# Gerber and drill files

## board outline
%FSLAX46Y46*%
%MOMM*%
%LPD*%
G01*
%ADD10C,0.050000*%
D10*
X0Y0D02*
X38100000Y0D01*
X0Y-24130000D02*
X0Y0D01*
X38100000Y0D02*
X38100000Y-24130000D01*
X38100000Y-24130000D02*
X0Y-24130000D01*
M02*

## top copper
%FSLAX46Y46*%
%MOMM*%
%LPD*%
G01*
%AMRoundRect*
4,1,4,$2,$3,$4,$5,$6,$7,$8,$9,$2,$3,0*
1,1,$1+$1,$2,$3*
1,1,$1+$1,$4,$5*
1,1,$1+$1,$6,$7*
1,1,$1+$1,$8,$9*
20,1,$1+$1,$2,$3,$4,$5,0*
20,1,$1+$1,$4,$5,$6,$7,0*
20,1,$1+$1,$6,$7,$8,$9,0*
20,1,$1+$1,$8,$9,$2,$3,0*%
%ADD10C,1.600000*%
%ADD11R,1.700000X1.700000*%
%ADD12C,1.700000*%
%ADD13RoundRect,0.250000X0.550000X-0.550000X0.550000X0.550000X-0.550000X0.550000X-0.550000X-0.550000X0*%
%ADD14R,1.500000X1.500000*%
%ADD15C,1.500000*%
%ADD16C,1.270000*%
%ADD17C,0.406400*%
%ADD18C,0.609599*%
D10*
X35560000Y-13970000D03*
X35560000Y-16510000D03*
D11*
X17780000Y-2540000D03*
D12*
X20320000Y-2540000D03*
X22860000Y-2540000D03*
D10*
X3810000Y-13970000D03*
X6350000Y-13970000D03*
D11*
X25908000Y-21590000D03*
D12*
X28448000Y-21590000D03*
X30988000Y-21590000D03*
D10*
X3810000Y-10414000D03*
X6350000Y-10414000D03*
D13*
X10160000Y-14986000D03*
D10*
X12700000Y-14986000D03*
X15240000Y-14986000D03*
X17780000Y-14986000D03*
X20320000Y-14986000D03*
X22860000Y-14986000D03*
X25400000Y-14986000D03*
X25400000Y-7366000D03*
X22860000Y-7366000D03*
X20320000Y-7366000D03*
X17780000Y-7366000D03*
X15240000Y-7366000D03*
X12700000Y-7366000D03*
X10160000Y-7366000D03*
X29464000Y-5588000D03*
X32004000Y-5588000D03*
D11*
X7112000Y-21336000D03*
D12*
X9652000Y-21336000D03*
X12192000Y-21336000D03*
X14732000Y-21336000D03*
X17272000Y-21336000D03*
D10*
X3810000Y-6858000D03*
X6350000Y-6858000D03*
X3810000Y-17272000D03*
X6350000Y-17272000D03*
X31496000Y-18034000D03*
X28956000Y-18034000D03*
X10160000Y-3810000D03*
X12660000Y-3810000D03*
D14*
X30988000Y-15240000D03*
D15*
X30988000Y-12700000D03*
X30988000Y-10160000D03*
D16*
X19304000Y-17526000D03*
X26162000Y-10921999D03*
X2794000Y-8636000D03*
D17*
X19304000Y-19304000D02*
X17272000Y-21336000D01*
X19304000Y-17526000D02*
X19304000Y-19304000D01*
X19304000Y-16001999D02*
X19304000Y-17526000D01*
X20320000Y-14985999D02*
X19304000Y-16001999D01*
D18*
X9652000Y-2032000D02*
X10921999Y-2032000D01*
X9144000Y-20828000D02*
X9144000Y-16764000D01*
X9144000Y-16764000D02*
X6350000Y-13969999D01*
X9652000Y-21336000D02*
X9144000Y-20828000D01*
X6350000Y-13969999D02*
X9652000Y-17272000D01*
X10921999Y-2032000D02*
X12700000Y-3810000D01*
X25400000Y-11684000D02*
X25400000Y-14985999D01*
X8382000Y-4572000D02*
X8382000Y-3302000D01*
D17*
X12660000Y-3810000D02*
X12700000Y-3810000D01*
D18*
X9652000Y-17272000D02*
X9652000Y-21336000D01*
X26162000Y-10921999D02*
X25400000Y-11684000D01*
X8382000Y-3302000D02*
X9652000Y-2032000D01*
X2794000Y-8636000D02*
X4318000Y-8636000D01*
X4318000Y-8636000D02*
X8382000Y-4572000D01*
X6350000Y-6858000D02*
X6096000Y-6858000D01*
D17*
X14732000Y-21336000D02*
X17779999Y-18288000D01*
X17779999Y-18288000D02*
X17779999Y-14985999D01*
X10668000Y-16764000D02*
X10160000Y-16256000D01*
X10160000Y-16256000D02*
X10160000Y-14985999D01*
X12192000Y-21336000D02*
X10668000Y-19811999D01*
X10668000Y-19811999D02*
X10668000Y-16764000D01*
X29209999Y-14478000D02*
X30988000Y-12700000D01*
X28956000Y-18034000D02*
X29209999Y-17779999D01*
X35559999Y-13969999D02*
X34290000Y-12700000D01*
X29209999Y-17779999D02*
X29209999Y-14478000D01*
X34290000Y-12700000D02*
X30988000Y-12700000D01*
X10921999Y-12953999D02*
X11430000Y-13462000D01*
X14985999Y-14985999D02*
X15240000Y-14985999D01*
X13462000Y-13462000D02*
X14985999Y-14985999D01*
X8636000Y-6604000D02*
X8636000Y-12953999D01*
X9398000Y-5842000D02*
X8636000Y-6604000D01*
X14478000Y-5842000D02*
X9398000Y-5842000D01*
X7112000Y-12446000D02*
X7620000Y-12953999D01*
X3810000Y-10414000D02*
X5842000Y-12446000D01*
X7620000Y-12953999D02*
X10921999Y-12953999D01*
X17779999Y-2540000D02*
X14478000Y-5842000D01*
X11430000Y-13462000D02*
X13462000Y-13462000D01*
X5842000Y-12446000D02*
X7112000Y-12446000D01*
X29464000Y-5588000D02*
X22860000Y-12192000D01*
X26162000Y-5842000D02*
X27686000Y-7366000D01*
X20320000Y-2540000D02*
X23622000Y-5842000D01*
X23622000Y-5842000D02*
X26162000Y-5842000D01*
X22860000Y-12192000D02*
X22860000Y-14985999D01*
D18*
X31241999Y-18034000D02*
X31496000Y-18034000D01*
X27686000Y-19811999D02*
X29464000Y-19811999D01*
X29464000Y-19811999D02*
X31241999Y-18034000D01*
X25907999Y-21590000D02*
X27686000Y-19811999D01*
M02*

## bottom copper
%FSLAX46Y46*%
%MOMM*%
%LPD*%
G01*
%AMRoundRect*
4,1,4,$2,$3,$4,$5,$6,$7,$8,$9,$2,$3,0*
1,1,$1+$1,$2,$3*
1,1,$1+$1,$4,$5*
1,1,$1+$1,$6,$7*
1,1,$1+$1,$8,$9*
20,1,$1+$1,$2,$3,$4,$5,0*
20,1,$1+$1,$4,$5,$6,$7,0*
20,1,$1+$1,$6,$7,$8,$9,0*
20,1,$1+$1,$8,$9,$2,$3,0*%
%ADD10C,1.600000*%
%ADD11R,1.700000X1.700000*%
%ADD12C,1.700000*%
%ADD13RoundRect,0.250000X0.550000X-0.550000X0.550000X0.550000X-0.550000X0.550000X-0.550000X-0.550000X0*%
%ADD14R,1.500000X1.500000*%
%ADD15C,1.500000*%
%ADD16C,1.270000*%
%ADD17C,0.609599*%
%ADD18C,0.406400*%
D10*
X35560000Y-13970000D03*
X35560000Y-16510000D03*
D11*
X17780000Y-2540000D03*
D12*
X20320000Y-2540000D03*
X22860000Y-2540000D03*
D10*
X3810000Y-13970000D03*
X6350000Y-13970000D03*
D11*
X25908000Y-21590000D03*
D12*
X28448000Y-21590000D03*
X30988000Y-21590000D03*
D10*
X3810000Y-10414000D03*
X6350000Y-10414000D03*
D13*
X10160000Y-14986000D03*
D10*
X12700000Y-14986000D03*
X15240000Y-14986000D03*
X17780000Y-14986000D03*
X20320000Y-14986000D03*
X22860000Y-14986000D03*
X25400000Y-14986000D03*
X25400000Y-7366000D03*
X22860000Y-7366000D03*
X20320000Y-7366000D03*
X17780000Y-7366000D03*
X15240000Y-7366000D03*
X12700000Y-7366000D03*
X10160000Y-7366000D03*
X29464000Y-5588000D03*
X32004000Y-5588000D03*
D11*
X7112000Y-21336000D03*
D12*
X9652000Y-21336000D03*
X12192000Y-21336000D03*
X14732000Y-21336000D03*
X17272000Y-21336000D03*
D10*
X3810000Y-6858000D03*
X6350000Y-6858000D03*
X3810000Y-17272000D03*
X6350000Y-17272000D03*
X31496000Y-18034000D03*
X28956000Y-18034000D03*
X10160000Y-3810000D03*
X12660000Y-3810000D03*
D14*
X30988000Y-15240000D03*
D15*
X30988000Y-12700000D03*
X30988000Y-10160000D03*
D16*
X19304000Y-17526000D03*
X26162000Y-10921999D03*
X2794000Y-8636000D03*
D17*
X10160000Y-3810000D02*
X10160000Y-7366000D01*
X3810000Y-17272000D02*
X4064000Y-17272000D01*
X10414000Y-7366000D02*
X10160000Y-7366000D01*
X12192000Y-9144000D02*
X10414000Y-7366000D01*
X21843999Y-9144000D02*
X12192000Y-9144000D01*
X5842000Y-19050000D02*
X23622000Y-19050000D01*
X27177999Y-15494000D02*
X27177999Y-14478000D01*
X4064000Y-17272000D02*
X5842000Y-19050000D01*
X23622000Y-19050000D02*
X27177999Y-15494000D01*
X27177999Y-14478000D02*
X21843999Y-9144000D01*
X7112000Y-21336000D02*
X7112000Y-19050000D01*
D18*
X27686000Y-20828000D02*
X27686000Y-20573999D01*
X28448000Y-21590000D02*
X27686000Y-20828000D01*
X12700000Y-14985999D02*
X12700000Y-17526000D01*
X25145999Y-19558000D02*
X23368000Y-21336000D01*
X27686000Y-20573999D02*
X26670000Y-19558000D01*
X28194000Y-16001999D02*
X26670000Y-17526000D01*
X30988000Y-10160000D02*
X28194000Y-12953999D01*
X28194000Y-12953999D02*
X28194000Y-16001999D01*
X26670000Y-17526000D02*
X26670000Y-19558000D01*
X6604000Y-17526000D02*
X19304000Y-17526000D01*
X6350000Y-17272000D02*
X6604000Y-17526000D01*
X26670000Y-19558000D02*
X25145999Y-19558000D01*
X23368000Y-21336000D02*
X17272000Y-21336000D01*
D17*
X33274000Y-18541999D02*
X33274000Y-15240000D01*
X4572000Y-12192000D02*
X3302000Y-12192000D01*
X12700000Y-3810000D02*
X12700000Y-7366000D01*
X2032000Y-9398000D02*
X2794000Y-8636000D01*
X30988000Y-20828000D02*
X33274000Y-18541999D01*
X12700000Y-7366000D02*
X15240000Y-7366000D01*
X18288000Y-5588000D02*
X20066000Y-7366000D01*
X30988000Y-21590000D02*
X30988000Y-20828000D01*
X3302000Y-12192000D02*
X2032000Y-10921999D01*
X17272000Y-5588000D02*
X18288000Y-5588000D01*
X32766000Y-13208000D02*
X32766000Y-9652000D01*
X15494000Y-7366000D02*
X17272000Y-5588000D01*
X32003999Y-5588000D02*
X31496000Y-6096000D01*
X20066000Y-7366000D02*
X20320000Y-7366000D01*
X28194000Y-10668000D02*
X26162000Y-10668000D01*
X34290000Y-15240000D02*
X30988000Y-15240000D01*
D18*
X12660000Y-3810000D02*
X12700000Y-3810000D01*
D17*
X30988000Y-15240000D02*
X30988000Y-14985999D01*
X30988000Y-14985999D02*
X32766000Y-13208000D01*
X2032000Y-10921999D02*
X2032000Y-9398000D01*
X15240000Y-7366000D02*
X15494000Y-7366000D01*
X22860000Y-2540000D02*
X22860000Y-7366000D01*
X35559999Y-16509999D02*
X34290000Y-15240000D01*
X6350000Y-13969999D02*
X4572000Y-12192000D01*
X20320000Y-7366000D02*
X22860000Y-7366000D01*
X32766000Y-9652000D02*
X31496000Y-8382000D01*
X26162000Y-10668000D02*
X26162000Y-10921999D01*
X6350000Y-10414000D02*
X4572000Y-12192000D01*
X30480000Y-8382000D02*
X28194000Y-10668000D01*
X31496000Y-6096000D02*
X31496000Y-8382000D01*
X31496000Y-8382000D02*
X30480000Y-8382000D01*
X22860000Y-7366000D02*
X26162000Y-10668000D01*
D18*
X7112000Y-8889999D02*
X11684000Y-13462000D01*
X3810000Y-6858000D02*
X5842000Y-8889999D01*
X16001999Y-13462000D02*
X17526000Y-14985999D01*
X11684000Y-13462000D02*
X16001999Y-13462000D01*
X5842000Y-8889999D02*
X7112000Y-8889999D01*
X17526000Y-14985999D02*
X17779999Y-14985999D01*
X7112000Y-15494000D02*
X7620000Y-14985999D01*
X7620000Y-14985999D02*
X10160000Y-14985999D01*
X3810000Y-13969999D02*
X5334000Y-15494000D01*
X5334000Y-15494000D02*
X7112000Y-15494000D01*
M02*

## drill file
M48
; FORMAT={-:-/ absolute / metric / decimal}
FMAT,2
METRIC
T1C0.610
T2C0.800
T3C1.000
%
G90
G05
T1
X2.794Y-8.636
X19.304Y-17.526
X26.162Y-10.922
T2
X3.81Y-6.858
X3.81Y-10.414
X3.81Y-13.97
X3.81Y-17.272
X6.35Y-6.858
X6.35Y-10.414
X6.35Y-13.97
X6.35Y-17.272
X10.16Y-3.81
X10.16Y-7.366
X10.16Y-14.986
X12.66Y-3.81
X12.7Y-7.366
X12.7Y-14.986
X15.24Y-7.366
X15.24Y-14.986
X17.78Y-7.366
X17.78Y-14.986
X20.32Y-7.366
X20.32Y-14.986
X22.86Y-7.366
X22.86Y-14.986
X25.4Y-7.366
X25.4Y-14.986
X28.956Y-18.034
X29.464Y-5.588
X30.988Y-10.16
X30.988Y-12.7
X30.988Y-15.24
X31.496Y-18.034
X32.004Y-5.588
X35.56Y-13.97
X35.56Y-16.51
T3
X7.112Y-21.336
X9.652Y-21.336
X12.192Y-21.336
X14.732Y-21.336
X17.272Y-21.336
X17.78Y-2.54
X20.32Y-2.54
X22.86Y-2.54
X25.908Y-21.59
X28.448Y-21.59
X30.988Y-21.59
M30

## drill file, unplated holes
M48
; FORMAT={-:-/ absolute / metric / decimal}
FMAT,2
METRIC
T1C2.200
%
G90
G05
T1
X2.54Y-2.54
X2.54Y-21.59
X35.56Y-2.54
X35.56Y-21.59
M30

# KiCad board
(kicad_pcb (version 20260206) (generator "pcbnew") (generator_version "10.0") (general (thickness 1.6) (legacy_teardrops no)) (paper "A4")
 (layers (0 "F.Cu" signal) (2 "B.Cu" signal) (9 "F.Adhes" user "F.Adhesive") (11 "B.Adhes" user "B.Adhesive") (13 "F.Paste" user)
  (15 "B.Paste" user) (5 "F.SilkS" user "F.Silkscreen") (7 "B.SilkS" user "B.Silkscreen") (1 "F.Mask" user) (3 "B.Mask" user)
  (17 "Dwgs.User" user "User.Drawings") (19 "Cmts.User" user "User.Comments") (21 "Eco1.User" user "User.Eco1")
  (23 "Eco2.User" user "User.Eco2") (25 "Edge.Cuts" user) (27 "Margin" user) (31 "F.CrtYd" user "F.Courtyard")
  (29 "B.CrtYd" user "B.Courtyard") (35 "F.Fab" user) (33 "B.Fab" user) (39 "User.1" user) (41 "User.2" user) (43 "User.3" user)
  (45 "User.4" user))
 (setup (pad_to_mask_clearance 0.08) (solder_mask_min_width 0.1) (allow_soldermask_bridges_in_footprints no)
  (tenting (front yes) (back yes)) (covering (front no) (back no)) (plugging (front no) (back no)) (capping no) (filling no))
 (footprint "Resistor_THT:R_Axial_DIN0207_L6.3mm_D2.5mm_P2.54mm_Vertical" (layer "F.Cu") (at 35.56 13.97 -90)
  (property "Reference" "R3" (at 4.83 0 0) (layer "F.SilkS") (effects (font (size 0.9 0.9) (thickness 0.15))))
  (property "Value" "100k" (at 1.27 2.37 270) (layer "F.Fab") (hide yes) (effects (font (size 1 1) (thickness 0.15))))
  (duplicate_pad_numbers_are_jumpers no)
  (pad "1" thru_hole circle (at 0 0 270) (size 1.6 1.6) (drill 0.8) (layers "*.Cu" "*.Mask") (remove_unused_layers no) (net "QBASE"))
  (pad "2" thru_hole circle (at 2.54 0 270) (size 1.6 1.6) (drill 0.8) (layers "*.Cu" "*.Mask") (remove_unused_layers no) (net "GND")))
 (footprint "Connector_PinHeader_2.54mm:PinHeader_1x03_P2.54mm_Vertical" (layer "F.Cu") (at 17.78 2.54 90)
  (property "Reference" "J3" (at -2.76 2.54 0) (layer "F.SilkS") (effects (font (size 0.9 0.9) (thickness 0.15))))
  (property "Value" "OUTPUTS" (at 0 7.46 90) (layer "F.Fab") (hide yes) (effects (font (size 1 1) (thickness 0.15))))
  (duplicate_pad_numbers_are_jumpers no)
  (pad "1" thru_hole rect (at 0 0 90) (size 1.7 1.7) (drill 1) (layers "*.Cu" "*.Mask") (remove_unused_layers no) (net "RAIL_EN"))
  (pad "2" thru_hole circle (at 0 2.54 90) (size 1.7 1.7) (drill 1) (layers "*.Cu" "*.Mask") (remove_unused_layers no) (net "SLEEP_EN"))
  (pad "3" thru_hole circle (at 0 5.08 90) (size 1.7 1.7) (drill 1) (layers "*.Cu" "*.Mask") (remove_unused_layers no) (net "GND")))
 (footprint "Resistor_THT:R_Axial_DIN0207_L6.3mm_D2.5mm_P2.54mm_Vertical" (layer "F.Cu") (at 3.81 13.97)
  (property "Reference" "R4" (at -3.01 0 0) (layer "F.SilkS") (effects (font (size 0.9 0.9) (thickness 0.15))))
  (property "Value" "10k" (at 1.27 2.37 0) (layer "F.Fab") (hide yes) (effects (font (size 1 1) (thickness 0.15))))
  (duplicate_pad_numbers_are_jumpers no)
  (pad "1" thru_hole circle (at 0 0) (size 1.6 1.6) (drill 0.8) (layers "*.Cu" "*.Mask") (remove_unused_layers no) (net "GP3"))
  (pad "2" thru_hole circle (at 2.54 0) (size 1.6 1.6) (drill 0.8) (layers "*.Cu" "*.Mask") (remove_unused_layers no) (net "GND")))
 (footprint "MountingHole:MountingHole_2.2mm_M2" (layer "F.Cu") (at 2.54 21.59)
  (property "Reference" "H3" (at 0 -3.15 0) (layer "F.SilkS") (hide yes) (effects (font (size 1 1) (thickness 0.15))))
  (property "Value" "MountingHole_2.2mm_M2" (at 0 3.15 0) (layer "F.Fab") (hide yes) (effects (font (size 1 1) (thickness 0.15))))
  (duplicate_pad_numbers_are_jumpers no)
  (pad "" np_thru_hole circle (at 0 0) (size 2.2 2.2) (drill 2.2) (layers "*.Cu" "*.Mask")))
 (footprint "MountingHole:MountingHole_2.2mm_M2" (layer "F.Cu") (at 35.56 2.54)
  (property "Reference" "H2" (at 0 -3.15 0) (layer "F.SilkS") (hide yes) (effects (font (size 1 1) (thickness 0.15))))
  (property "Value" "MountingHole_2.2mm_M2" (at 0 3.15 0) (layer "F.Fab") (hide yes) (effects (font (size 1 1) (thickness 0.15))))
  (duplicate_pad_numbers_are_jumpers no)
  (pad "" np_thru_hole circle (at 0 0) (size 2.2 2.2) (drill 2.2) (layers "*.Cu" "*.Mask")))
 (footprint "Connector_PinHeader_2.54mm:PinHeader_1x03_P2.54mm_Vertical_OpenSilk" (layer "F.Cu") (at 25.908 21.59 90)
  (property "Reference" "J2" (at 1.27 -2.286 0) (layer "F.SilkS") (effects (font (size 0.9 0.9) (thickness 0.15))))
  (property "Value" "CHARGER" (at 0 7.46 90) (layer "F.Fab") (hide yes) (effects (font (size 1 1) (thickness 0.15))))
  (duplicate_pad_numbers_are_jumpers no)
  (pad "1" thru_hole rect (at 0 0 90) (size 1.7 1.7) (drill 1) (layers "*.Cu" "*.Mask") (remove_unused_layers no) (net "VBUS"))
  (pad "2" thru_hole circle (at 0 2.54 90) (size 1.7 1.7) (drill 1) (layers "*.Cu" "*.Mask") (remove_unused_layers no) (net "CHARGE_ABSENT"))
  (pad "3" thru_hole circle (at 0 5.08 90) (size 1.7 1.7) (drill 1) (layers "*.Cu" "*.Mask") (remove_unused_layers no) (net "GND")))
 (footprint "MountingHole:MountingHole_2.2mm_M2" (layer "F.Cu") (at 2.54 2.54)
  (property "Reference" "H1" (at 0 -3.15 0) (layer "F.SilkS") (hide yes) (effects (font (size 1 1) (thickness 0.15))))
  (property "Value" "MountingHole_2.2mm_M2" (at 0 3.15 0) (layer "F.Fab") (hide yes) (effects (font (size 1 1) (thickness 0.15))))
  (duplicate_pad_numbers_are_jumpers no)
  (pad "" np_thru_hole circle (at 0 0) (size 2.2 2.2) (drill 2.2) (layers "*.Cu" "*.Mask")))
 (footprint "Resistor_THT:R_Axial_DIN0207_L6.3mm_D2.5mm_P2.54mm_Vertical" (layer "F.Cu") (at 3.81 10.414)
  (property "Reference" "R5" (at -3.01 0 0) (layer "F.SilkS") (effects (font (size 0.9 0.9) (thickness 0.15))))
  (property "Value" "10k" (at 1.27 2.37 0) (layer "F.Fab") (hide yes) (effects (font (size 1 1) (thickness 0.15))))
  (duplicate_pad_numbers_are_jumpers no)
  (pad "1" thru_hole circle (at 0 0) (size 1.6 1.6) (drill 0.8) (layers "*.Cu" "*.Mask") (remove_unused_layers no) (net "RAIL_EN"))
  (pad "2" thru_hole circle (at 2.54 0) (size 1.6 1.6) (drill 0.8) (layers "*.Cu" "*.Mask") (remove_unused_layers no) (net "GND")))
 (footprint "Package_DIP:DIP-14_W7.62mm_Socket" (layer "F.Cu") (at 10.16 14.986 90)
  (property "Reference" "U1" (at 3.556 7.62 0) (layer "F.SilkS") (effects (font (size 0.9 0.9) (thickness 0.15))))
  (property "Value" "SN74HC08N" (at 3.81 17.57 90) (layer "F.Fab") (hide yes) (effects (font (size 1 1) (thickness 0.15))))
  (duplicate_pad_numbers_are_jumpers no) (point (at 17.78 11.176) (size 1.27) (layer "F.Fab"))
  (pad "1" thru_hole roundrect (at 0 0 90) (size 1.6 1.6) (drill 0.8) (layers "*.Cu" "*.Mask") (remove_unused_layers no)
   (roundrect_rratio 0.15625) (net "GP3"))
  (pad "2" thru_hole circle (at 0 2.54 90) (size 1.6 1.6) (drill 0.8) (layers "*.Cu" "*.Mask") (remove_unused_layers no)
   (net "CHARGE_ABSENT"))
  (pad "3" thru_hole circle (at 0 5.08 90) (size 1.6 1.6) (drill 0.8) (layers "*.Cu" "*.Mask") (remove_unused_layers no) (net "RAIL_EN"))
  (pad "4" thru_hole circle (at 0 7.62 90) (size 1.6 1.6) (drill 0.8) (layers "*.Cu" "*.Mask") (remove_unused_layers no) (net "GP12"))
  (pad "5" thru_hole circle (at 0 10.16 90) (size 1.6 1.6) (drill 0.8) (layers "*.Cu" "*.Mask") (remove_unused_layers no)
   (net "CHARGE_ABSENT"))
  (pad "6" thru_hole circle (at 0 12.7 90) (size 1.6 1.6) (drill 0.8) (layers "*.Cu" "*.Mask") (remove_unused_layers no) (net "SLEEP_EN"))
  (pad "7" thru_hole circle (at 0 15.24 90) (size 1.6 1.6) (drill 0.8) (layers "*.Cu" "*.Mask") (remove_unused_layers no) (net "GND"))
  (pad "8" thru_hole circle (at 7.62 15.24 90) (size 1.6 1.6) (drill 0.8) (layers "*.Cu" "*.Mask") (remove_unused_layers no) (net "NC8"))
  (pad "9" thru_hole circle (at 7.62 12.7 90) (size 1.6 1.6) (drill 0.8) (layers "*.Cu" "*.Mask") (remove_unused_layers no) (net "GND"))
  (pad "10" thru_hole circle (at 7.62 10.16 90) (size 1.6 1.6) (drill 0.8) (layers "*.Cu" "*.Mask") (remove_unused_layers no) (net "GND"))
  (pad "11" thru_hole circle (at 7.62 7.62 90) (size 1.6 1.6) (drill 0.8) (layers "*.Cu" "*.Mask") (remove_unused_layers no) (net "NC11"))
  (pad "12" thru_hole circle (at 7.62 5.08 90) (size 1.6 1.6) (drill 0.8) (layers "*.Cu" "*.Mask") (remove_unused_layers no) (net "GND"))
  (pad "13" thru_hole circle (at 7.62 2.54 90) (size 1.6 1.6) (drill 0.8) (layers "*.Cu" "*.Mask") (remove_unused_layers no) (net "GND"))
  (pad "14" thru_hole circle (at 7.62 0 90) (size 1.6 1.6) (drill 0.8) (layers "*.Cu" "*.Mask") (remove_unused_layers no) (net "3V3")))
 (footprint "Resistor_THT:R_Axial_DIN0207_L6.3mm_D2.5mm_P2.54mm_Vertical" (layer "F.Cu") (at 29.464 5.588)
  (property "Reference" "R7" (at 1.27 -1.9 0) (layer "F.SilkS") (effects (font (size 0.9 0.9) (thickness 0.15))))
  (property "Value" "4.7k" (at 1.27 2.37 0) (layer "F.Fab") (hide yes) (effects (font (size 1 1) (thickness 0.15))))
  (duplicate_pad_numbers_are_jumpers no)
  (pad "1" thru_hole circle (at 0 0) (size 1.6 1.6) (drill 0.8) (layers "*.Cu" "*.Mask") (remove_unused_layers no) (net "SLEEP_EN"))
  (pad "2" thru_hole circle (at 2.54 0) (size 1.6 1.6) (drill 0.8) (layers "*.Cu" "*.Mask") (remove_unused_layers no) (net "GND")))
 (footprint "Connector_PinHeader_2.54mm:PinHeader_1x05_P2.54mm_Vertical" (layer "F.Cu") (at 7.112 21.336 90)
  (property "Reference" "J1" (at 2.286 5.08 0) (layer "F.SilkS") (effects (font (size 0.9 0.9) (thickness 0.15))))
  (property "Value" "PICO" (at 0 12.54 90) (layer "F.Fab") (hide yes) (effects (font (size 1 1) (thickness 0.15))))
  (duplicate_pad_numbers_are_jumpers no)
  (pad "1" thru_hole rect (at 0 0 90) (size 1.7 1.7) (drill 1) (layers "*.Cu" "*.Mask") (remove_unused_layers no) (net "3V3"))
  (pad "2" thru_hole circle (at 0 2.54 90) (size 1.7 1.7) (drill 1) (layers "*.Cu" "*.Mask") (remove_unused_layers no) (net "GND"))
  (pad "3" thru_hole circle (at 0 5.08 90) (size 1.7 1.7) (drill 1) (layers "*.Cu" "*.Mask") (remove_unused_layers no) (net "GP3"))
  (pad "4" thru_hole circle (at 0 7.62 90) (size 1.7 1.7) (drill 1) (layers "*.Cu" "*.Mask") (remove_unused_layers no) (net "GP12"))
  (pad "5" thru_hole circle (at 0 10.16 90) (size 1.7 1.7) (drill 1) (layers "*.Cu" "*.Mask") (remove_unused_layers no)
   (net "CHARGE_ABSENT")))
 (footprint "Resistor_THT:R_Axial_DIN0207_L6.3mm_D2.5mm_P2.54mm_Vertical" (layer "F.Cu") (at 3.81 6.858)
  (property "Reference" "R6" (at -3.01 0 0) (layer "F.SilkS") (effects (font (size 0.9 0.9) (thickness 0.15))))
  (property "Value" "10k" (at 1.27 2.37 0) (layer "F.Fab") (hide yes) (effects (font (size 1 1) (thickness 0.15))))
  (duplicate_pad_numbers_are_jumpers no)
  (pad "1" thru_hole circle (at 0 0) (size 1.6 1.6) (drill 0.8) (layers "*.Cu" "*.Mask") (remove_unused_layers no) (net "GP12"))
  (pad "2" thru_hole circle (at 2.54 0) (size 1.6 1.6) (drill 0.8) (layers "*.Cu" "*.Mask") (remove_unused_layers no) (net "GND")))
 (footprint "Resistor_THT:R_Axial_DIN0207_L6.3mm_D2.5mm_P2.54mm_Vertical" (layer "F.Cu") (at 3.81 17.272)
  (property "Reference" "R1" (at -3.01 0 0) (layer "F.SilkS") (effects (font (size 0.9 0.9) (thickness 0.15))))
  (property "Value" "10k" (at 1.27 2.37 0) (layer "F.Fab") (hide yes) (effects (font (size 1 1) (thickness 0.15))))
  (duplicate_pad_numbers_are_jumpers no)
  (pad "1" thru_hole circle (at 0 0) (size 1.6 1.6) (drill 0.8) (layers "*.Cu" "*.Mask") (remove_unused_layers no) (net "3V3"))
  (pad "2" thru_hole circle (at 2.54 0) (size 1.6 1.6) (drill 0.8) (layers "*.Cu" "*.Mask") (remove_unused_layers no) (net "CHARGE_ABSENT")))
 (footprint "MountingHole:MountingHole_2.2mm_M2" (layer "F.Cu") (at 35.56 21.59)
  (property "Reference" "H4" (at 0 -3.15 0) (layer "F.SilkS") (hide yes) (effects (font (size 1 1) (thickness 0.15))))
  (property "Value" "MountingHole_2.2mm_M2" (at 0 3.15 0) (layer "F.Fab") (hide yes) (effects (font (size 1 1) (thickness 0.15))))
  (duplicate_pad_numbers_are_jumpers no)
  (pad "" np_thru_hole circle (at 0 0) (size 2.2 2.2) (drill 2.2) (layers "*.Cu" "*.Mask")))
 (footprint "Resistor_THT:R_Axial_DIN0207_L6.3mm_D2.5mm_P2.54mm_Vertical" (layer "F.Cu") (at 31.496 18.034 180)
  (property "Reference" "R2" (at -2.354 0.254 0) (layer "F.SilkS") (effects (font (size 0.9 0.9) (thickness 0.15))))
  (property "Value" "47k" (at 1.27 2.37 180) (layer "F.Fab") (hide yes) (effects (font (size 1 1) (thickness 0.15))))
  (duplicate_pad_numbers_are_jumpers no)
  (pad "1" thru_hole circle (at 0 0 180) (size 1.6 1.6) (drill 0.8) (layers "*.Cu" "*.Mask") (remove_unused_layers no) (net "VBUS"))
  (pad "2" thru_hole circle (at 2.54 0 180) (size 1.6 1.6) (drill 0.8) (layers "*.Cu" "*.Mask") (remove_unused_layers no) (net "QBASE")))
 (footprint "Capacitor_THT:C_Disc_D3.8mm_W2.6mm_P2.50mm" (layer "F.Cu") (at 10.16 3.81)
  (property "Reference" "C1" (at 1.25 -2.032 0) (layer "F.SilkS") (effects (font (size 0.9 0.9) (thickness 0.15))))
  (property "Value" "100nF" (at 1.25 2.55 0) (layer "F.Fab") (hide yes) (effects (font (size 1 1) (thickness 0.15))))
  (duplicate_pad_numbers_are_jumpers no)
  (pad "1" thru_hole circle (at 0 0) (size 1.6 1.6) (drill 0.8) (layers "*.Cu" "*.Mask") (remove_unused_layers no) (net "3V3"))
  (pad "2" thru_hole circle (at 2.5 0) (size 1.6 1.6) (drill 0.8) (layers "*.Cu" "*.Mask") (remove_unused_layers no) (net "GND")))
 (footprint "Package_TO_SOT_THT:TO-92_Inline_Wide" (layer "F.Cu") (at 30.988 15.24 90)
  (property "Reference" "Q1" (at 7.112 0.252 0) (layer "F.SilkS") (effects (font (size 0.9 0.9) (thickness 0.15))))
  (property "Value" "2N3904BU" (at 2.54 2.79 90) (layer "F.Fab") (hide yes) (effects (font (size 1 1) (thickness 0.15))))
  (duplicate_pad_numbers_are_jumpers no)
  (pad "1" thru_hole rect (at 0 0 90) (size 1.5 1.5) (drill 0.8) (layers "*.Cu" "*.Mask") (remove_unused_layers no) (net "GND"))
  (pad "2" thru_hole circle (at 2.54 0 90) (size 1.5 1.5) (drill 0.8) (layers "*.Cu" "*.Mask") (remove_unused_layers no) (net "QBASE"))
  (pad "3" thru_hole circle (at 5.08 0 90) (size 1.5 1.5) (drill 0.8) (layers "*.Cu" "*.Mask") (remove_unused_layers no)
   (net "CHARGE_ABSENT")))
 (gr_line (start 0 0) (end 38.1 0) (stroke (width 0.05) (type default)) (layer "Edge.Cuts"))
 (gr_line (start 0 24.13) (end 0 0) (stroke (width 0.05) (type default)) (layer "Edge.Cuts"))
 (gr_line (start 38.1 0) (end 38.1 24.13) (stroke (width 0.05) (type default)) (layer "Edge.Cuts"))
 (gr_line (start 38.1 24.13) (end 0 24.13) (stroke (width 0.05) (type default)) (layer "Edge.Cuts"))
 (segment (start 10.16 3.81) (end 10.16 7.366) (width 0.609599) (layer "B.Cu") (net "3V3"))
 (segment (start 3.81 17.272) (end 4.064 17.272) (width 0.609599) (layer "B.Cu") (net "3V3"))
 (segment (start 10.414 7.366) (end 10.16 7.366) (width 0.609599) (layer "B.Cu") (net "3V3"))
 (segment (start 12.192 9.144) (end 10.414 7.366) (width 0.609599) (layer "B.Cu") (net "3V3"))
 (segment (start 21.843999 9.144) (end 12.192 9.144) (width 0.609599) (layer "B.Cu") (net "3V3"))
 (segment (start 5.842 19.05) (end 23.622 19.05) (width 0.609599) (layer "B.Cu") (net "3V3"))
 (segment (start 27.177999 15.494) (end 27.177999 14.478) (width 0.609599) (layer "B.Cu") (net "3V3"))
 (segment (start 4.064 17.272) (end 5.842 19.05) (width 0.609599) (layer "B.Cu") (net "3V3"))
 (segment (start 23.622 19.05) (end 27.177999 15.494) (width 0.609599) (layer "B.Cu") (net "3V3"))
 (segment (start 27.177999 14.478) (end 21.843999 9.144) (width 0.609599) (layer "B.Cu") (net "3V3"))
 (segment (start 7.112 21.336) (end 7.112 19.05) (width 0.609599) (layer "B.Cu") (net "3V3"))
 (segment (start 19.304 19.304) (end 17.272 21.336) (width 0.4064) (layer "F.Cu") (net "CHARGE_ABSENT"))
 (segment (start 19.304 17.526) (end 19.304 19.304) (width 0.4064) (layer "F.Cu") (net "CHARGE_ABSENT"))
 (segment (start 19.304 16.001999) (end 19.304 17.526) (width 0.4064) (layer "F.Cu") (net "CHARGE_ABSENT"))
 (segment (start 20.32 14.985999) (end 19.304 16.001999) (width 0.4064) (layer "F.Cu") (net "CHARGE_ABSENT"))
 (via (at 19.304 17.526) (size 1.27) (drill 0.6096) (layers "F.Cu" "B.Cu") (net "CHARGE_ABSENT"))
 (segment (start 27.686 20.828) (end 27.686 20.573999) (width 0.4064) (layer "B.Cu") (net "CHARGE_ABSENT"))
 (segment (start 28.448 21.59) (end 27.686 20.828) (width 0.4064) (layer "B.Cu") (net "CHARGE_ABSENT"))
 (segment (start 12.7 14.985999) (end 12.7 17.526) (width 0.4064) (layer "B.Cu") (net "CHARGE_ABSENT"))
 (segment (start 25.145999 19.558) (end 23.368 21.336) (width 0.4064) (layer "B.Cu") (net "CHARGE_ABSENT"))
 (segment (start 27.686 20.573999) (end 26.67 19.558) (width 0.4064) (layer "B.Cu") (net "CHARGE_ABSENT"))
 (segment (start 28.194 16.001999) (end 26.67 17.526) (width 0.4064) (layer "B.Cu") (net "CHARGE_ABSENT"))
 (segment (start 30.988 10.16) (end 28.194 12.953999) (width 0.4064) (layer "B.Cu") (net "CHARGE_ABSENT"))
 (segment (start 28.194 12.953999) (end 28.194 16.001999) (width 0.4064) (layer "B.Cu") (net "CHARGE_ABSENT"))
 (segment (start 26.67 17.526) (end 26.67 19.558) (width 0.4064) (layer "B.Cu") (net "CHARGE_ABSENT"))
 (segment (start 6.604 17.526) (end 19.304 17.526) (width 0.4064) (layer "B.Cu") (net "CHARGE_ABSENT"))
 (segment (start 6.35 17.272) (end 6.604 17.526) (width 0.4064) (layer "B.Cu") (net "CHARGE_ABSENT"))
 (segment (start 26.67 19.558) (end 25.145999 19.558) (width 0.4064) (layer "B.Cu") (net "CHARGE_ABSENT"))
 (segment (start 23.368 21.336) (end 17.272 21.336) (width 0.4064) (layer "B.Cu") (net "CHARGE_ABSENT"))
 (segment (start 9.652 2.032) (end 10.921999 2.032) (width 0.609599) (layer "F.Cu") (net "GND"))
 (segment (start 9.144 20.828) (end 9.144 16.764) (width 0.609599) (layer "F.Cu") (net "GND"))
 (segment (start 9.144 16.764) (end 6.35 13.969999) (width 0.609599) (layer "F.Cu") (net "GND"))
 (segment (start 9.652 21.336) (end 9.144 20.828) (width 0.609599) (layer "F.Cu") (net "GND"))
 (segment (start 6.35 13.969999) (end 9.652 17.272) (width 0.609599) (layer "F.Cu") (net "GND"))
 (segment (start 10.921999 2.032) (end 12.7 3.81) (width 0.609599) (layer "F.Cu") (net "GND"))
 (segment (start 25.4 11.684) (end 25.4 14.985999) (width 0.609599) (layer "F.Cu") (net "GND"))
 (segment (start 8.382 4.572) (end 8.382 3.302) (width 0.609599) (layer "F.Cu") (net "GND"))
 (segment (start 12.66 3.81) (end 12.7 3.81) (width 0.4064) (layer "F.Cu") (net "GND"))
 (segment (start 9.652 17.272) (end 9.652 21.336) (width 0.609599) (layer "F.Cu") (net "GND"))
 (segment (start 26.162 10.921999) (end 25.4 11.684) (width 0.609599) (layer "F.Cu") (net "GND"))
 (segment (start 8.382 3.302) (end 9.652 2.032) (width 0.609599) (layer "F.Cu") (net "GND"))
 (segment (start 2.794 8.636) (end 4.318 8.636) (width 0.609599) (layer "F.Cu") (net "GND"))
 (segment (start 4.318 8.636) (end 8.382 4.572) (width 0.609599) (layer "F.Cu") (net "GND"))
 (segment (start 6.35 6.858) (end 6.096 6.858) (width 0.609599) (layer "F.Cu") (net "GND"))
 (via (at 26.162 10.921999) (size 1.27) (drill 0.6096) (layers "F.Cu" "B.Cu") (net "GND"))
 (via (at 2.794 8.636) (size 1.27) (drill 0.6096) (layers "F.Cu" "B.Cu") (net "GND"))
 (segment (start 33.274 18.541999) (end 33.274 15.24) (width 0.609599) (layer "B.Cu") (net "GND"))
 (segment (start 4.572 12.192) (end 3.302 12.192) (width 0.609599) (layer "B.Cu") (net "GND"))
 (segment (start 12.7 3.81) (end 12.7 7.366) (width 0.609599) (layer "B.Cu") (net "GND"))
 (segment (start 2.032 9.398) (end 2.794 8.636) (width 0.609599) (layer "B.Cu") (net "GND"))
 (segment (start 30.988 20.828) (end 33.274 18.541999) (width 0.609599) (layer "B.Cu") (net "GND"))
 (segment (start 12.7 7.366) (end 15.24 7.366) (width 0.609599) (layer "B.Cu") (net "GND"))
 (segment (start 18.288 5.588) (end 20.066 7.366) (width 0.609599) (layer "B.Cu") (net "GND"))
 (segment (start 30.988 21.59) (end 30.988 20.828) (width 0.609599) (layer "B.Cu") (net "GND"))
 (segment (start 3.302 12.192) (end 2.032 10.921999) (width 0.609599) (layer "B.Cu") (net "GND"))
 (segment (start 17.272 5.588) (end 18.288 5.588) (width 0.609599) (layer "B.Cu") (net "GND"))
 (segment (start 32.766 13.208) (end 32.766 9.652) (width 0.609599) (layer "B.Cu") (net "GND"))
 (segment (start 15.494 7.366) (end 17.272 5.588) (width 0.609599) (layer "B.Cu") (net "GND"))
 (segment (start 32.003999 5.588) (end 31.496 6.096) (width 0.609599) (layer "B.Cu") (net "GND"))
 (segment (start 20.066 7.366) (end 20.32 7.366) (width 0.609599) (layer "B.Cu") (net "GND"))
 (segment (start 28.194 10.668) (end 26.162 10.668) (width 0.609599) (layer "B.Cu") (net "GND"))
 (segment (start 34.29 15.24) (end 30.988 15.24) (width 0.609599) (layer "B.Cu") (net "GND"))
 (segment (start 12.66 3.81) (end 12.7 3.81) (width 0.4064) (layer "B.Cu") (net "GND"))
 (segment (start 30.988 15.24) (end 30.988 14.985999) (width 0.609599) (layer "B.Cu") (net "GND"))
 (segment (start 30.988 14.985999) (end 32.766 13.208) (width 0.609599) (layer "B.Cu") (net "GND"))
 (segment (start 2.032 10.921999) (end 2.032 9.398) (width 0.609599) (layer "B.Cu") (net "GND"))
 (segment (start 15.24 7.366) (end 15.494 7.366) (width 0.609599) (layer "B.Cu") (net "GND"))
 (segment (start 22.86 2.54) (end 22.86 7.366) (width 0.609599) (layer "B.Cu") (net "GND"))
 (segment (start 35.559999 16.509999) (end 34.29 15.24) (width 0.609599) (layer "B.Cu") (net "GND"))
 (segment (start 6.35 13.969999) (end 4.572 12.192) (width 0.609599) (layer "B.Cu") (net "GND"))
 (segment (start 20.32 7.366) (end 22.86 7.366) (width 0.609599) (layer "B.Cu") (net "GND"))
 (segment (start 32.766 9.652) (end 31.496 8.382) (width 0.609599) (layer "B.Cu") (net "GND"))
 (segment (start 26.162 10.668) (end 26.162 10.921999) (width 0.609599) (layer "B.Cu") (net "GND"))
 (segment (start 6.35 10.414) (end 4.572 12.192) (width 0.609599) (layer "B.Cu") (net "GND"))
 (segment (start 30.48 8.382) (end 28.194 10.668) (width 0.609599) (layer "B.Cu") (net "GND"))
 (segment (start 31.496 6.096) (end 31.496 8.382) (width 0.609599) (layer "B.Cu") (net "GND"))
 (segment (start 31.496 8.382) (end 30.48 8.382) (width 0.609599) (layer "B.Cu") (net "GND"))
 (segment (start 22.86 7.366) (end 26.162 10.668) (width 0.609599) (layer "B.Cu") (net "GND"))
 (segment (start 14.732 21.336) (end 17.779999 18.288) (width 0.4064) (layer "F.Cu") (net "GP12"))
 (segment (start 17.779999 18.288) (end 17.779999 14.985999) (width 0.4064) (layer "F.Cu") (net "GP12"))
 (segment (start 7.112 8.889999) (end 11.684 13.462) (width 0.4064) (layer "B.Cu") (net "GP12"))
 (segment (start 3.81 6.858) (end 5.842 8.889999) (width 0.4064) (layer "B.Cu") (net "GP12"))
 (segment (start 16.001999 13.462) (end 17.526 14.985999) (width 0.4064) (layer "B.Cu") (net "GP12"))
 (segment (start 11.684 13.462) (end 16.001999 13.462) (width 0.4064) (layer "B.Cu") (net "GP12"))
 (segment (start 5.842 8.889999) (end 7.112 8.889999) (width 0.4064) (layer "B.Cu") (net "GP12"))
 (segment (start 17.526 14.985999) (end 17.779999 14.985999) (width 0.4064) (layer "B.Cu") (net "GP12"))
 (segment (start 10.668 16.764) (end 10.16 16.256) (width 0.4064) (layer "F.Cu") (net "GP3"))
 (segment (start 10.16 16.256) (end 10.16 14.985999) (width 0.4064) (layer "F.Cu") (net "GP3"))
 (segment (start 12.192 21.336) (end 10.668 19.811999) (width 0.4064) (layer "F.Cu") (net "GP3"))
 (segment (start 10.668 19.811999) (end 10.668 16.764) (width 0.4064) (layer "F.Cu") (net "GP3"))
 (segment (start 7.112 15.494) (end 7.62 14.985999) (width 0.4064) (layer "B.Cu") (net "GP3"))
 (segment (start 7.62 14.985999) (end 10.16 14.985999) (width 0.4064) (layer "B.Cu") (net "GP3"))
 (segment (start 3.81 13.969999) (end 5.334 15.494) (width 0.4064) (layer "B.Cu") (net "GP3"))
 (segment (start 5.334 15.494) (end 7.112 15.494) (width 0.4064) (layer "B.Cu") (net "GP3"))
 (segment (start 29.209999 14.478) (end 30.988 12.7) (width 0.4064) (layer "F.Cu") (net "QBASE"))
 (segment (start 28.956 18.034) (end 29.209999 17.779999) (width 0.4064) (layer "F.Cu") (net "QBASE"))
 (segment (start 35.559999 13.969999) (end 34.29 12.7) (width 0.4064) (layer "F.Cu") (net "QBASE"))
 (segment (start 29.209999 17.779999) (end 29.209999 14.478) (width 0.4064) (layer "F.Cu") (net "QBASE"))
 (segment (start 34.29 12.7) (end 30.988 12.7) (width 0.4064) (layer "F.Cu") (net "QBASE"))
 (segment (start 10.921999 12.953999) (end 11.43 13.462) (width 0.4064) (layer "F.Cu") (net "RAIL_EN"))
 (segment (start 14.985999 14.985999) (end 15.24 14.985999) (width 0.4064) (layer "F.Cu") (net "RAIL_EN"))
 (segment (start 13.462 13.462) (end 14.985999 14.985999) (width 0.4064) (layer "F.Cu") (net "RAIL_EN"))
 (segment (start 8.636 6.604) (end 8.636 12.953999) (width 0.4064) (layer "F.Cu") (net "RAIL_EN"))
 (segment (start 9.398 5.842) (end 8.636 6.604) (width 0.4064) (layer "F.Cu") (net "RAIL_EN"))
 (segment (start 14.478 5.842) (end 9.398 5.842) (width 0.4064) (layer "F.Cu") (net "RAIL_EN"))
 (segment (start 7.112 12.446) (end 7.62 12.953999) (width 0.4064) (layer "F.Cu") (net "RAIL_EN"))
 (segment (start 3.81 10.414) (end 5.842 12.446) (width 0.4064) (layer "F.Cu") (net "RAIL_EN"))
 (segment (start 7.62 12.953999) (end 10.921999 12.953999) (width 0.4064) (layer "F.Cu") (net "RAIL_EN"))
 (segment (start 17.779999 2.54) (end 14.478 5.842) (width 0.4064) (layer "F.Cu") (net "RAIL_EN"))
 (segment (start 11.43 13.462) (end 13.462 13.462) (width 0.4064) (layer "F.Cu") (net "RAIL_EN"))
 (segment (start 5.842 12.446) (end 7.112 12.446) (width 0.4064) (layer "F.Cu") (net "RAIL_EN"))
 (segment (start 29.464 5.588) (end 22.86 12.192) (width 0.4064) (layer "F.Cu") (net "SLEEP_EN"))
 (segment (start 26.162 5.842) (end 27.686 7.366) (width 0.4064) (layer "F.Cu") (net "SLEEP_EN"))
 (segment (start 20.32 2.54) (end 23.622 5.842) (width 0.4064) (layer "F.Cu") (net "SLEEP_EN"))
 (segment (start 23.622 5.842) (end 26.162 5.842) (width 0.4064) (layer "F.Cu") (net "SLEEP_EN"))
 (segment (start 22.86 12.192) (end 22.86 14.985999) (width 0.4064) (layer "F.Cu") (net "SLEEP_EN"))
 (segment (start 31.241999 18.034) (end 31.496 18.034) (width 0.609599) (layer "F.Cu") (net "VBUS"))
 (segment (start 27.686 19.811999) (end 29.464 19.811999) (width 0.609599) (layer "F.Cu") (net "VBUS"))
 (segment (start 29.464 19.811999) (end 31.241999 18.034) (width 0.609599) (layer "F.Cu") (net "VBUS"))
 (segment (start 25.907999 21.59) (end 27.686 19.811999) (width 0.609599) (layer "F.Cu") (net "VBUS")))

